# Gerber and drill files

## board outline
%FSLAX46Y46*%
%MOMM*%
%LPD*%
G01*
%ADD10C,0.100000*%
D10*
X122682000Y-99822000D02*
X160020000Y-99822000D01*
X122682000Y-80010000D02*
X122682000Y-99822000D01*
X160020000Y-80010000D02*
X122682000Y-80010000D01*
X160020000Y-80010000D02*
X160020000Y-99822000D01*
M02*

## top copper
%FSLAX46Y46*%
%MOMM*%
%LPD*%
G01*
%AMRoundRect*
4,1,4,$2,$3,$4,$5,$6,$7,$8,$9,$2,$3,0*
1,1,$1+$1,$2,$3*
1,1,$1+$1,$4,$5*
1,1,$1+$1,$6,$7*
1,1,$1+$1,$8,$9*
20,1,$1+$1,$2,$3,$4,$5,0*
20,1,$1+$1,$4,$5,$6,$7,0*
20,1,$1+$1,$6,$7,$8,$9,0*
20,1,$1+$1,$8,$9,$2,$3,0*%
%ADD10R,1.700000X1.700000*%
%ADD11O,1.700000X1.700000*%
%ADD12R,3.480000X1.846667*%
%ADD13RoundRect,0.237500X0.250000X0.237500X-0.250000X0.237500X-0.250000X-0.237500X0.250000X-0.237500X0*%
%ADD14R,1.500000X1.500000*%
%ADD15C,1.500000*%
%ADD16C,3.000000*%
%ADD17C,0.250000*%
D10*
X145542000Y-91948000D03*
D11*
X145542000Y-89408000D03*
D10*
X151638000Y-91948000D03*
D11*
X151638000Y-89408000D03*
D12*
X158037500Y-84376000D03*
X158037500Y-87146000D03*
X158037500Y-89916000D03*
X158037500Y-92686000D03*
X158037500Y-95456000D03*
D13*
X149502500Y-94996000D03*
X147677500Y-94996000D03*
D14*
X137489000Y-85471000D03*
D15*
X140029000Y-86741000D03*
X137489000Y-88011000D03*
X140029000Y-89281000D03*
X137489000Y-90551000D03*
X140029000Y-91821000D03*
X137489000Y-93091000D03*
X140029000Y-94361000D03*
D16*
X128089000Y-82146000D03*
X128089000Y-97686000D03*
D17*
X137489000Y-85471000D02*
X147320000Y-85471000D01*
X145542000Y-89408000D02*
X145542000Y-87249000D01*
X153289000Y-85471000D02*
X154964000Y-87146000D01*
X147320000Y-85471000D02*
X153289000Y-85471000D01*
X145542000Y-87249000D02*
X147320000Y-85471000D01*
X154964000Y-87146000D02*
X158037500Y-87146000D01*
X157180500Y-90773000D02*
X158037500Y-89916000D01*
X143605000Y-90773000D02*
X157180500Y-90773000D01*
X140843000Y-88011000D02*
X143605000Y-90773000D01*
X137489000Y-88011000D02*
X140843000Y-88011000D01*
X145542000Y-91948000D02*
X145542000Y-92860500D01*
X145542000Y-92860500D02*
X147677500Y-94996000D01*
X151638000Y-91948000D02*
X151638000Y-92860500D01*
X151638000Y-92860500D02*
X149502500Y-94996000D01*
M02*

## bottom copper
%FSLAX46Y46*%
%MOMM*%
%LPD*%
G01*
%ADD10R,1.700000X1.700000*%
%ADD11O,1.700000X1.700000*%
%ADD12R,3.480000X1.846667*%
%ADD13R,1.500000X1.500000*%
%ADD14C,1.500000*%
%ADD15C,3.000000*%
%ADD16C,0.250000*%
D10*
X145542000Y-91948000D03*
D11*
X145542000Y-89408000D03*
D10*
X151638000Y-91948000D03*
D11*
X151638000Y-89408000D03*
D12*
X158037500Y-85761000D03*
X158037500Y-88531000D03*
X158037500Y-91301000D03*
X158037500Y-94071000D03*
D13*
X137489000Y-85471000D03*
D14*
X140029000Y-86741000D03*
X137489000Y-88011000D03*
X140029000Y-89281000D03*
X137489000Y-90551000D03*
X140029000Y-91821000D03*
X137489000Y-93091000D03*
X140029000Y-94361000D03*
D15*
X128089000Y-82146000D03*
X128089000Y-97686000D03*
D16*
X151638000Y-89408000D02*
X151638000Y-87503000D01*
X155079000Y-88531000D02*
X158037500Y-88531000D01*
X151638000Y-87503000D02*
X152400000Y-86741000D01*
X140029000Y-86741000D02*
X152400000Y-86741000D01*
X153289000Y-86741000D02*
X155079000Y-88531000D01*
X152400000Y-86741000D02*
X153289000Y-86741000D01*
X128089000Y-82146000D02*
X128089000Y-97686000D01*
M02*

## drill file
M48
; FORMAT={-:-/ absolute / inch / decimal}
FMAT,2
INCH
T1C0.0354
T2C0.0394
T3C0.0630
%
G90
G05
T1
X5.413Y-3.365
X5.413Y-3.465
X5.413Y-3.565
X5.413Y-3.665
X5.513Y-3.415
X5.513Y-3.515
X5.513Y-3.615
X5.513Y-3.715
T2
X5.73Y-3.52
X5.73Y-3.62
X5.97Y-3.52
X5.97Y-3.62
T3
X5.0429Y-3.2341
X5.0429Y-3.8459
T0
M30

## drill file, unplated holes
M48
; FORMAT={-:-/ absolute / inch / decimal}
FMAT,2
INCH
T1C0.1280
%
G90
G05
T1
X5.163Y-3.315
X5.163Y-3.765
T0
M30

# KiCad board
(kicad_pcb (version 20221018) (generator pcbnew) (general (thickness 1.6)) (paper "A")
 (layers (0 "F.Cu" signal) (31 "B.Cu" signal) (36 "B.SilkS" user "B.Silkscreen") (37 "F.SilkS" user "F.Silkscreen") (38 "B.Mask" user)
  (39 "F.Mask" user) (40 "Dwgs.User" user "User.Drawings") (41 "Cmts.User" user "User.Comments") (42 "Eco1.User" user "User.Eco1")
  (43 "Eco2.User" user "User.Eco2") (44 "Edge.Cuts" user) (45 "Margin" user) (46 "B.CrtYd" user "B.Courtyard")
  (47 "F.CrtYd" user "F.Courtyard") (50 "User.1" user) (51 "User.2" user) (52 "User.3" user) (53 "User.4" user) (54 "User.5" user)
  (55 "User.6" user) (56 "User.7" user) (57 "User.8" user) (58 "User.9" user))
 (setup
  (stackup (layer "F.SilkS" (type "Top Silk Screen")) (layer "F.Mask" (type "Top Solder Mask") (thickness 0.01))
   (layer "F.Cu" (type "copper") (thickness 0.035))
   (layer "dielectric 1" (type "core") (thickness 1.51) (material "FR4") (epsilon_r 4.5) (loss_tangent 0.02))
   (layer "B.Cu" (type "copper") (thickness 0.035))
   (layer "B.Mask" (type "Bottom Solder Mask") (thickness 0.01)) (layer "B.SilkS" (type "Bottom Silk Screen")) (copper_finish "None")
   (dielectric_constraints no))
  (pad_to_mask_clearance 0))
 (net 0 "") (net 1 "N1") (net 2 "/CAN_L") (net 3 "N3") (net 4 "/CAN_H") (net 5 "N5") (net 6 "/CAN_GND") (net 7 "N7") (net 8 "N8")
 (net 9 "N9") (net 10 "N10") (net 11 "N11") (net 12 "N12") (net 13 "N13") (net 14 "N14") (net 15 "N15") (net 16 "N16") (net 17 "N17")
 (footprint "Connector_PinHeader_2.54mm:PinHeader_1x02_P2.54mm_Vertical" (layer "F.Cu") (at 145.542 91.948 180)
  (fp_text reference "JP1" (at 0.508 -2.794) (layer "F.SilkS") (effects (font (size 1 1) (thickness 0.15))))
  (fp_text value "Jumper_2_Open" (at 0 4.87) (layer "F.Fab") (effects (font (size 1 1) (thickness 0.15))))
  (pad "1" thru_hole rect (at 0 0 180) (size 1.7 1.7) (drill 1) (layers "*.Cu" "*.Mask") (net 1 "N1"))
  (pad "2" thru_hole oval (at 0 2.54 180) (size 1.7 1.7) (drill 1) (layers "*.Cu" "*.Mask") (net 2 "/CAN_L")))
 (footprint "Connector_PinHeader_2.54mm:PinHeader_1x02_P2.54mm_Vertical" (layer "F.Cu") (at 151.638 91.948 180)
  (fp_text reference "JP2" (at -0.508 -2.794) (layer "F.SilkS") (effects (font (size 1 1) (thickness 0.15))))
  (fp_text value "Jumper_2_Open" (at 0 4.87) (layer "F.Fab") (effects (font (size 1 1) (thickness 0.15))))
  (pad "1" thru_hole rect (at 0 0 180) (size 1.7 1.7) (drill 1) (layers "*.Cu" "*.Mask") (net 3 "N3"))
  (pad "2" thru_hole oval (at 0 2.54 180) (size 1.7 1.7) (drill 1) (layers "*.Cu" "*.Mask") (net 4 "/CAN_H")))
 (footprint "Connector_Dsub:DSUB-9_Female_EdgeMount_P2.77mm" (layer "F.Cu") (at 158.0375 89.916 90)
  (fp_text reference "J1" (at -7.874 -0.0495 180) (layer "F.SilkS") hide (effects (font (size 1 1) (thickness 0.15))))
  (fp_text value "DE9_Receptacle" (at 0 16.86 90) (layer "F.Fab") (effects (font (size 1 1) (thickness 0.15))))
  (pad "1" smd rect (at 5.54 0 90) (size 1.846667 3.48) (layers "F.Cu" "F.Paste" "F.Mask") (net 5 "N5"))
  (pad "2" smd rect (at 2.77 0 90) (size 1.846667 3.48) (layers "F.Cu" "F.Paste" "F.Mask") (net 2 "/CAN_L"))
  (pad "3" smd rect (at 0 0 90) (size 1.846667 3.48) (layers "F.Cu" "F.Paste" "F.Mask") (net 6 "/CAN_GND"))
  (pad "4" smd rect (at -2.77 0 90) (size 1.846667 3.48) (layers "F.Cu" "F.Paste" "F.Mask") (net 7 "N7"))
  (pad "5" smd rect (at -5.54 0 90) (size 1.846667 3.48) (layers "F.Cu" "F.Paste" "F.Mask") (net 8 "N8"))
  (pad "6" smd rect (at 4.155 0 90) (size 1.846667 3.48) (layers "B.Cu" "B.Paste" "B.Mask") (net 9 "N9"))
  (pad "7" smd rect (at 1.385 0 90) (size 1.846667 3.48) (layers "B.Cu" "B.Paste" "B.Mask") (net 4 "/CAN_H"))
  (pad "8" smd rect (at -1.385 0 90) (size 1.846667 3.48) (layers "B.Cu" "B.Paste" "B.Mask") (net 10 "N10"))
  (pad "9" smd rect (at -4.155 0 90) (size 1.846667 3.48) (layers "B.Cu" "B.Paste" "B.Mask") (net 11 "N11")))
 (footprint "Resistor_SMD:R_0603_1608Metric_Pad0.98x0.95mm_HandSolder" (layer "F.Cu") (at 148.59 94.996 180)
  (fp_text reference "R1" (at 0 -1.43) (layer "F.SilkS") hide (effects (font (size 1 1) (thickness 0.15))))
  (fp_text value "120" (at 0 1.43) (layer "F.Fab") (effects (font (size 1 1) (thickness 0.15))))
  (pad "1" smd roundrect (at -0.9125 0 180) (size 0.975 0.95) (layers "F.Cu" "F.Paste" "F.Mask") (roundrect_rratio 0.25) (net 3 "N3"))
  (pad "2" smd roundrect (at 0.9125 0 180) (size 0.975 0.95) (layers "F.Cu" "F.Paste" "F.Mask") (roundrect_rratio 0.25) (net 1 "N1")))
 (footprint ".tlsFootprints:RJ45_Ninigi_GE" (layer "F.Cu") (at 137.489 85.471 -90)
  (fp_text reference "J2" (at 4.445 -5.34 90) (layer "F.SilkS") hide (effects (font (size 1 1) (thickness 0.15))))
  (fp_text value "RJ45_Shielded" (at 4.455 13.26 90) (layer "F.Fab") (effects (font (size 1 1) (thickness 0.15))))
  (pad "" np_thru_hole circle (at -1.27 6.35 270) (size 3.25 3.25) (drill 3.25) (layers "*.Cu" "*.Mask"))
  (pad "" np_thru_hole circle (at 10.16 6.35 90) (size 3.25 3.25) (drill 3.25) (layers "*.Cu" "*.Mask"))
  (pad "1" thru_hole rect (at 0 0 90) (size 1.5 1.5) (drill 0.9) (layers "*.Cu" "*.Mask") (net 2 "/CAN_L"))
  (pad "2" thru_hole circle (at 1.27 -2.54 90) (size 1.5 1.5) (drill 0.9) (layers "*.Cu" "*.Mask") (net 4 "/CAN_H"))
  (pad "3" thru_hole circle (at 2.54 0 90) (size 1.5 1.5) (drill 0.9) (layers "*.Cu" "*.Mask") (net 6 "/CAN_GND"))
  (pad "4" thru_hole circle (at 3.81 -2.54 90) (size 1.5 1.5) (drill 0.9) (layers "*.Cu" "*.Mask") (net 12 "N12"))
  (pad "5" thru_hole circle (at 5.08 0 90) (size 1.5 1.5) (drill 0.9) (layers "*.Cu" "*.Mask") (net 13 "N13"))
  (pad "6" thru_hole circle (at 6.35 -2.54 90) (size 1.5 1.5) (drill 0.9) (layers "*.Cu" "*.Mask") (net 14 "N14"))
  (pad "7" thru_hole circle (at 7.62 0 90) (size 1.5 1.5) (drill 0.9) (layers "*.Cu" "*.Mask") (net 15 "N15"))
  (pad "8" thru_hole circle (at 8.89 -2.54 90) (size 1.5 1.5) (drill 0.9) (layers "*.Cu" "*.Mask") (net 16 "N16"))
  (pad "SH" thru_hole circle (at -3.325 9.4 270) (size 3 3) (drill 1.6) (layers "*.Cu" "*.Mask") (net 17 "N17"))
  (pad "SH" thru_hole circle (at 12.215 9.4 90) (size 3 3) (drill 1.6) (layers "*.Cu" "*.Mask") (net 17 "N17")))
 (gr_line (start 122.682 99.822) (end 160.02 99.822) (stroke (width 0.1) (type default)) (layer "Edge.Cuts"))
 (gr_line (start 122.682 80.01) (end 122.682 99.822) (stroke (width 0.1) (type default)) (layer "Edge.Cuts"))
 (gr_line (start 160.02 80.01) (end 122.682 80.01) (stroke (width 0.1) (type default)) (layer "Edge.Cuts"))
 (gr_line (start 160.02 80.01) (end 160.02 99.822) (stroke (width 0.1) (type default)) (layer "Edge.Cuts"))
 (segment (start 137.489 85.471) (end 147.32 85.471) (width 0.25) (layer "F.Cu") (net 2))
 (segment (start 145.542 89.408) (end 145.542 87.249) (width 0.25) (layer "F.Cu") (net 2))
 (segment (start 153.289 85.471) (end 154.964 87.146) (width 0.25) (layer "F.Cu") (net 2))
 (segment (start 147.32 85.471) (end 153.289 85.471) (width 0.25) (layer "F.Cu") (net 2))
 (segment (start 145.542 87.249) (end 147.32 85.471) (width 0.25) (layer "F.Cu") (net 2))
 (segment (start 154.964 87.146) (end 158.0375 87.146) (width 0.25) (layer "F.Cu") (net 2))
 (segment (start 157.1805 90.773) (end 158.0375 89.916) (width 0.25) (layer "F.Cu") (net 6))
 (segment (start 143.605 90.773) (end 157.1805 90.773) (width 0.25) (layer "F.Cu") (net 6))
 (segment (start 140.843 88.011) (end 143.605 90.773) (width 0.25) (layer "F.Cu") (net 6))
 (segment (start 137.489 88.011) (end 140.843 88.011) (width 0.25) (layer "F.Cu") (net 6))
 (segment (start 151.638 89.408) (end 151.638 87.503) (width 0.25) (layer "B.Cu") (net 4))
 (segment (start 155.079 88.531) (end 158.0375 88.531) (width 0.25) (layer "B.Cu") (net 4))
 (segment (start 151.638 87.503) (end 152.4 86.741) (width 0.25) (layer "B.Cu") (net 4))
 (segment (start 140.029 86.741) (end 152.4 86.741) (width 0.25) (layer "B.Cu") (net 4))
 (segment (start 153.289 86.741) (end 155.079 88.531) (width 0.25) (layer "B.Cu") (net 4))
 (segment (start 152.4 86.741) (end 153.289 86.741) (width 0.25) (layer "B.Cu") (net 4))
 (segment (start 145.542 91.948) (end 145.542 92.8605) (width 0.25) (layer "F.Cu") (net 1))
 (segment (start 145.542 92.8605) (end 147.6775 94.996) (width 0.25) (layer "F.Cu") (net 1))
 (segment (start 151.638 91.948) (end 151.638 92.8605) (width 0.25) (layer "F.Cu") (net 3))
 (segment (start 151.638 92.8605) (end 149.5025 94.996) (width 0.25) (layer "F.Cu") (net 3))
 (segment (start 128.089 82.146) (end 128.089 97.686) (width 0.25) (layer "B.Cu") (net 17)))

